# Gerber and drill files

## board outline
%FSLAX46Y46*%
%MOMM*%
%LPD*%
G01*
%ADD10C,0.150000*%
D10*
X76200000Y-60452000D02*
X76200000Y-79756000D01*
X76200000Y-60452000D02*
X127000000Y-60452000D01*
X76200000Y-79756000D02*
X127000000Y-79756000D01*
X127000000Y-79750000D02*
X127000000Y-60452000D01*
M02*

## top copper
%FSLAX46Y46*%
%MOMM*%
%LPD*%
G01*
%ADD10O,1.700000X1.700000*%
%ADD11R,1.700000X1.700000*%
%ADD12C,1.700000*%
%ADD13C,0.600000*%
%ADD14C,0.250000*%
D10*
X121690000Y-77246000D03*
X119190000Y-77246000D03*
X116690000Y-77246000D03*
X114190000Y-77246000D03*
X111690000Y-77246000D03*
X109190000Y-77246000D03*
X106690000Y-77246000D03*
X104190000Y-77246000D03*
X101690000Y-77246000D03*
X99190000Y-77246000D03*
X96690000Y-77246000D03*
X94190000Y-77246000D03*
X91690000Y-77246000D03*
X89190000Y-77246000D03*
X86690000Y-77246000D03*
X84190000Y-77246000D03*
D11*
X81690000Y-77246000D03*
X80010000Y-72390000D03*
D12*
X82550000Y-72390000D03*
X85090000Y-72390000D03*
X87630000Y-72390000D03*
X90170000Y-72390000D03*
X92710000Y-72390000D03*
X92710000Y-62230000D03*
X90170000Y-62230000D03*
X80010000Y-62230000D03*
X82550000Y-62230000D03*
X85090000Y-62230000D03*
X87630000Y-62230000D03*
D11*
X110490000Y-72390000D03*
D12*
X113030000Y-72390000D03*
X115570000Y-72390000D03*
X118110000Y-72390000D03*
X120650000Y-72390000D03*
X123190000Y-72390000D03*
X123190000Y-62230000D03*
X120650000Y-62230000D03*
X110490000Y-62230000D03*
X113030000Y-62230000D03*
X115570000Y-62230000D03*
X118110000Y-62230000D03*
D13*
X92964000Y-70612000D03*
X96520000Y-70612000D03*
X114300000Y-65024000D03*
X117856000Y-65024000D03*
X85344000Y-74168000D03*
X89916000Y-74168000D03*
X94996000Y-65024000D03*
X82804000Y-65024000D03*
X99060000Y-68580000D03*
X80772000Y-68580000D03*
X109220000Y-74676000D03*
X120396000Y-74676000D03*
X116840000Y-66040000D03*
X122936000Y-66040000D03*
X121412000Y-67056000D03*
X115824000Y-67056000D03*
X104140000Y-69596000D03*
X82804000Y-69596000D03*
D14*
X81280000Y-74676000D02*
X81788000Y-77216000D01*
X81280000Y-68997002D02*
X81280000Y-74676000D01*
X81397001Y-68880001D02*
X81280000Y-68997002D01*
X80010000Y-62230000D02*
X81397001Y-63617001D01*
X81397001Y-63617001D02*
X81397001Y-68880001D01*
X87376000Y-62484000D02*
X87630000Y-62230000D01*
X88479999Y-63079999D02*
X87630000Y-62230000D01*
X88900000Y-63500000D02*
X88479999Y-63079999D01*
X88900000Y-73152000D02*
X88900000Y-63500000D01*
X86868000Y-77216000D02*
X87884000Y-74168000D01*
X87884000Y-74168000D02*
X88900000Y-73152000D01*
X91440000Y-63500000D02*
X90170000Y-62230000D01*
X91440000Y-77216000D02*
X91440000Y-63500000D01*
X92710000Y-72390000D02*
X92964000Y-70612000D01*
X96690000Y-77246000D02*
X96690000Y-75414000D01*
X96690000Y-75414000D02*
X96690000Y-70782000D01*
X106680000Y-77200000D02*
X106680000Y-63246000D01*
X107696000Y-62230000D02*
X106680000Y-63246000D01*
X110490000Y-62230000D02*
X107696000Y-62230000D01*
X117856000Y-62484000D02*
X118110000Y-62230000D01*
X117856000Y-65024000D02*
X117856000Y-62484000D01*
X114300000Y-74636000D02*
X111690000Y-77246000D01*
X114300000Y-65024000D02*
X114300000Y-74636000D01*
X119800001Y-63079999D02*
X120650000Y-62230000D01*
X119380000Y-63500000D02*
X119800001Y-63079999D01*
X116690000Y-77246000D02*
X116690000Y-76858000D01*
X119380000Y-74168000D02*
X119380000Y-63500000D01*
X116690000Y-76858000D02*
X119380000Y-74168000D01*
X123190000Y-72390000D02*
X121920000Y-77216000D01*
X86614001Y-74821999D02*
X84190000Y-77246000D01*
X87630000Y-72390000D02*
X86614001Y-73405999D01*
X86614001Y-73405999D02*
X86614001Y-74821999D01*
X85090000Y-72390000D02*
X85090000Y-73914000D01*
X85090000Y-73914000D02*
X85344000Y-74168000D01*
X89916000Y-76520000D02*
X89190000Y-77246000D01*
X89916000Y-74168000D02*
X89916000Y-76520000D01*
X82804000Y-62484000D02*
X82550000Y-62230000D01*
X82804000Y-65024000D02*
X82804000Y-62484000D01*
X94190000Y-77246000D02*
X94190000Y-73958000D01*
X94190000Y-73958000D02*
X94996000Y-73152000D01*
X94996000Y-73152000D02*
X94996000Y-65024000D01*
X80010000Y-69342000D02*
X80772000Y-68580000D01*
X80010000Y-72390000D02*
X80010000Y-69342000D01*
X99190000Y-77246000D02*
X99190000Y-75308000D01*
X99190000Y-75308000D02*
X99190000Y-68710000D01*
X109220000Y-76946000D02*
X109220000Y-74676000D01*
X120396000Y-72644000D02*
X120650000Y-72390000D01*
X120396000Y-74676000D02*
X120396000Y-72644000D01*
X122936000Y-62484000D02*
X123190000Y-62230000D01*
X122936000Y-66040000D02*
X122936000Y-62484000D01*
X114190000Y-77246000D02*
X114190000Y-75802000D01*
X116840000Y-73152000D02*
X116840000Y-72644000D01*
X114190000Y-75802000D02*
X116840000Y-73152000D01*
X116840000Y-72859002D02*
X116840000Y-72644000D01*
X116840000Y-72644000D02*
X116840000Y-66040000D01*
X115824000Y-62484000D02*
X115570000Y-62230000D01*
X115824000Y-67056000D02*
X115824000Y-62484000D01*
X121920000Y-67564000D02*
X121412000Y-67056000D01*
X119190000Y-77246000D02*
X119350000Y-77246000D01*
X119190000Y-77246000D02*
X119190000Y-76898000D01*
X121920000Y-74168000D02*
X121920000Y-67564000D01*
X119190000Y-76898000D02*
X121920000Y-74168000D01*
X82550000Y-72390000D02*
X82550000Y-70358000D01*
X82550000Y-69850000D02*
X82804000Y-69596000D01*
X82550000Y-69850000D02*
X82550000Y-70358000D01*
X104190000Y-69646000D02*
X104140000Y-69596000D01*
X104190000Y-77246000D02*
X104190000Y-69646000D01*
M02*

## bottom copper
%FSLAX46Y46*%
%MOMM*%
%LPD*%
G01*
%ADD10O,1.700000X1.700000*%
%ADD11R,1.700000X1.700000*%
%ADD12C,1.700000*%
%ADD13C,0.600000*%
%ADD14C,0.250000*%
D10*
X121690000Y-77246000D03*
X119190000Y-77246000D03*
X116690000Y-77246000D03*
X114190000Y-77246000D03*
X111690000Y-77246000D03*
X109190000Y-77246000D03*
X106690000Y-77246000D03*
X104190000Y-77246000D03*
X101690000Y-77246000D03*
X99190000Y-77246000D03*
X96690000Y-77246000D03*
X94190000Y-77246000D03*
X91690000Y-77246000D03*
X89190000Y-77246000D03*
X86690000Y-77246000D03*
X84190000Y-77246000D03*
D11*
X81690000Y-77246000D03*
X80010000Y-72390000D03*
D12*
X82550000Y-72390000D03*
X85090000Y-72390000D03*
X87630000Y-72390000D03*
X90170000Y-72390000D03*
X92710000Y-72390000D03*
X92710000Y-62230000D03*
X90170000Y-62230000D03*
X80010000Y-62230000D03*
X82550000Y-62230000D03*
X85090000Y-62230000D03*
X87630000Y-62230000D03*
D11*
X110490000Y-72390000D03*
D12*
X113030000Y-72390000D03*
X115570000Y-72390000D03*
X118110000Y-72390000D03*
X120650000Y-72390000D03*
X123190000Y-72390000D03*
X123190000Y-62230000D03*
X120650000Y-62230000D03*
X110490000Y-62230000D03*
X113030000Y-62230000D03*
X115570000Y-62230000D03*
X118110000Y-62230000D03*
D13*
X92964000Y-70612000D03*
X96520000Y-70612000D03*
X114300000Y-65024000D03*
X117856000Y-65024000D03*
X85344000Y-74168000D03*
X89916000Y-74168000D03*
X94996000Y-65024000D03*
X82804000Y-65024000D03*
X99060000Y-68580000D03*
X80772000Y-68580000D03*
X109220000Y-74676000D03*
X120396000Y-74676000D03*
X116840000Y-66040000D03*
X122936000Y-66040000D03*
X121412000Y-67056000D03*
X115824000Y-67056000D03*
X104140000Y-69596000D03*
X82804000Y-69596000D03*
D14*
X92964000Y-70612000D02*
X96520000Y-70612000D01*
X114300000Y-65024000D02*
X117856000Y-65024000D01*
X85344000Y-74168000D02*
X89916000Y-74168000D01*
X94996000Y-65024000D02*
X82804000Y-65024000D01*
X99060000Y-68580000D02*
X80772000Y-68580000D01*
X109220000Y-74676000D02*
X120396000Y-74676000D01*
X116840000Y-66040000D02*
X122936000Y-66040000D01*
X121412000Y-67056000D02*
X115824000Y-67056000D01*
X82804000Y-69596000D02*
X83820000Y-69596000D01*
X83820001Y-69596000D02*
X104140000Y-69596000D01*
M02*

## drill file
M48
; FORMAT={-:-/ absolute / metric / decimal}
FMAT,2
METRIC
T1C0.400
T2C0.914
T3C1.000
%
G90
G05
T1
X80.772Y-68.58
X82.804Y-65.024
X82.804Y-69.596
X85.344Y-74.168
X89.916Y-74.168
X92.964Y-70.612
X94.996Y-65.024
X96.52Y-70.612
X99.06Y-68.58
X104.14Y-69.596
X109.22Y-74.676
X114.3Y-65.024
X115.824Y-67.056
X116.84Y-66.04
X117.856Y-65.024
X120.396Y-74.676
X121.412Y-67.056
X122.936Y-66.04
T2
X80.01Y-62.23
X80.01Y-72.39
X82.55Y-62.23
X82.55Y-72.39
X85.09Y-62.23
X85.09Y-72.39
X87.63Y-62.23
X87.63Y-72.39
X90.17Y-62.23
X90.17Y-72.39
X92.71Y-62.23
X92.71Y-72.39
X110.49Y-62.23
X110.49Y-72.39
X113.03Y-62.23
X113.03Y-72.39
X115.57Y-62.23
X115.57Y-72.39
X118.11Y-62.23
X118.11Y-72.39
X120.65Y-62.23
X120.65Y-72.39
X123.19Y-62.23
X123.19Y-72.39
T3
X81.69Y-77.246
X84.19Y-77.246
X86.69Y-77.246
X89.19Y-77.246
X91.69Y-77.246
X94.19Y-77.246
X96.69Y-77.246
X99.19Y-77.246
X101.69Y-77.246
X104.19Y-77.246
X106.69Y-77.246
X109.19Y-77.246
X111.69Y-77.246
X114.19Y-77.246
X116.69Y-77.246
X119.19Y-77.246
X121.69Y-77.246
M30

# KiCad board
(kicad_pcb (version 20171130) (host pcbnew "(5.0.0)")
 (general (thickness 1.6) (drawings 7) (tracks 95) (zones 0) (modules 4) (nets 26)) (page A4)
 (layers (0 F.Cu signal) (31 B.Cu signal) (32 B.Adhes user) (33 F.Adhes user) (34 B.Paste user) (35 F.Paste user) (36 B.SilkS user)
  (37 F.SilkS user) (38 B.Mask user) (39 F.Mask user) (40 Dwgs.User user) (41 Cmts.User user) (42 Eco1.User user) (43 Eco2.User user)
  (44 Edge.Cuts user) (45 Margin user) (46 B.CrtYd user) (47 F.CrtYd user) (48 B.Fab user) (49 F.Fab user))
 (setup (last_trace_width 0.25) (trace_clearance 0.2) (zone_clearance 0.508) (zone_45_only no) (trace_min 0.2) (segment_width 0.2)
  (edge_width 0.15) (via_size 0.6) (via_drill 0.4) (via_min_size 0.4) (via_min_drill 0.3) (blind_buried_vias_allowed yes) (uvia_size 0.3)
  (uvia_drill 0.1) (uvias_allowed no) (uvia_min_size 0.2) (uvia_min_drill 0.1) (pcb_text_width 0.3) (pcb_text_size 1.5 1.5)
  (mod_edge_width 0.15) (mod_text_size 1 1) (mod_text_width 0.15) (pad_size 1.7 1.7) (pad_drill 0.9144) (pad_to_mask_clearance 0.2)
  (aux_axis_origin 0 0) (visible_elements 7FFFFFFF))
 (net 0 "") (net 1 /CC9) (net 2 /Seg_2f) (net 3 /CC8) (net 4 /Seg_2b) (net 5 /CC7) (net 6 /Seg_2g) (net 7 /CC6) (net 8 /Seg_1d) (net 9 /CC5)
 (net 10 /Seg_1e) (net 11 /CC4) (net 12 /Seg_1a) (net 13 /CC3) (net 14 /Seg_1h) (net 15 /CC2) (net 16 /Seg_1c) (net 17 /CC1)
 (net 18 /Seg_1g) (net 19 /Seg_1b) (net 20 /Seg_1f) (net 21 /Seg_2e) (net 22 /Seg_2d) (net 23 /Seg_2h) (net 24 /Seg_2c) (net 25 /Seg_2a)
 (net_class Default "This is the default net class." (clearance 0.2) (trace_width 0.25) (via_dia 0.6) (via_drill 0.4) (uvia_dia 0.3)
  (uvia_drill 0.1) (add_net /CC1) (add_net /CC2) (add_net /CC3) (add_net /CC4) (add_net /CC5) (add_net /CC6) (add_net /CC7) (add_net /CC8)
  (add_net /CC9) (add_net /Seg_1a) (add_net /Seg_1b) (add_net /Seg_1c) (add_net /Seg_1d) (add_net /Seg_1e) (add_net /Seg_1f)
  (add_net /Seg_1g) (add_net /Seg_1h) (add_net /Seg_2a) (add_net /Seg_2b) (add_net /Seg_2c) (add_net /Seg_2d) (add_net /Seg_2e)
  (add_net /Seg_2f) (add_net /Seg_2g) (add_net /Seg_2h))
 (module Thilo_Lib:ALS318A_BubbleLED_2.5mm (layer F.Cu) (at 102.87 77.216)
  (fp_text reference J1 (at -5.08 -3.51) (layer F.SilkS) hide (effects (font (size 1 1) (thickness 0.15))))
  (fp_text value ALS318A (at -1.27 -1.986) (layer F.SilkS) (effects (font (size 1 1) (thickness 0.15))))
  (pad 17 thru_hole oval (at 18.82 0.03 90) (size 1.7 1.7) (drill 1) (layers *.Cu *.Mask) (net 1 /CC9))
  (pad 16 thru_hole oval (at 16.32 0.03 90) (size 1.7 1.7) (drill 1) (layers *.Cu *.Mask) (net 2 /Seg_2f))
  (pad 15 thru_hole oval (at 13.82 0.03 90) (size 1.7 1.7) (drill 1) (layers *.Cu *.Mask) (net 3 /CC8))
  (pad 14 thru_hole oval (at 11.32 0.03 90) (size 1.7 1.7) (drill 1) (layers *.Cu *.Mask) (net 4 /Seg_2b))
  (pad 13 thru_hole oval (at 8.82 0.03 90) (size 1.7 1.7) (drill 1) (layers *.Cu *.Mask) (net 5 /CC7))
  (pad 12 thru_hole oval (at 6.32 0.03 90) (size 1.7 1.7) (drill 1) (layers *.Cu *.Mask) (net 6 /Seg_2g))
  (pad 11 thru_hole oval (at 3.82 0.03 90) (size 1.7 1.7) (drill 1) (layers *.Cu *.Mask) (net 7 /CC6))
  (pad 10 thru_hole oval (at 1.32 0.03 90) (size 1.7 1.7) (drill 1) (layers *.Cu *.Mask) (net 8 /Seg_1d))
  (pad 9 thru_hole oval (at -1.18 0.03 90) (size 1.7 1.7) (drill 1) (layers *.Cu *.Mask) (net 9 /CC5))
  (pad 8 thru_hole oval (at -3.68 0.03 90) (size 1.7 1.7) (drill 1) (layers *.Cu *.Mask) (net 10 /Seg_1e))
  (pad 7 thru_hole oval (at -6.18 0.03 90) (size 1.7 1.7) (drill 1) (layers *.Cu *.Mask) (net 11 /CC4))
  (pad 6 thru_hole oval (at -8.68 0.03 90) (size 1.7 1.7) (drill 1) (layers *.Cu *.Mask) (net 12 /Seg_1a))
  (pad 5 thru_hole oval (at -11.18 0.03 90) (size 1.7 1.7) (drill 1) (layers *.Cu *.Mask) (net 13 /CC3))
  (pad 4 thru_hole oval (at -13.68 0.03 90) (size 1.7 1.7) (drill 1) (layers *.Cu *.Mask) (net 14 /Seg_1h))
  (pad 3 thru_hole oval (at -16.18 0.03 90) (size 1.7 1.7) (drill 1) (layers *.Cu *.Mask) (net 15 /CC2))
  (pad 2 thru_hole oval (at -18.68 0.03 90) (size 1.7 1.7) (drill 1) (layers *.Cu *.Mask) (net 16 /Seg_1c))
  (pad 1 thru_hole rect (at -21.18 0.03 90) (size 1.7 1.7) (drill 1) (layers *.Cu *.Mask) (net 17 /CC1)))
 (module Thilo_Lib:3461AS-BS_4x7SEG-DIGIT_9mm (layer F.Cu) (at 86.36 67.31)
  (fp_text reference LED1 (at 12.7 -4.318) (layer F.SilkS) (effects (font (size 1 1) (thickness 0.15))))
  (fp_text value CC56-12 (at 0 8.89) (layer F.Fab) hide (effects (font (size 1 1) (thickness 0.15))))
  (pad 1 thru_hole rect (at -6.35 5.08) (size 1.7 1.7) (drill 0.9144) (layers *.Cu *.Mask) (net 10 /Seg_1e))
  (pad 2 thru_hole circle (at -3.81 5.08) (size 1.7 1.7) (drill 0.9144) (layers *.Cu *.Mask) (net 8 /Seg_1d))
  (pad 3 thru_hole circle (at -1.27 5.08) (size 1.7 1.7) (drill 0.9144) (layers *.Cu *.Mask) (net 14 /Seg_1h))
  (pad 4 thru_hole circle (at 1.27 5.08) (size 1.7 1.7) (drill 0.9144) (layers *.Cu *.Mask) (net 16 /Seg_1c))
  (pad 5 thru_hole circle (at 3.81 5.08) (size 1.7 1.7) (drill 0.9144) (layers *.Cu *.Mask) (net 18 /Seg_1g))
  (pad 6 thru_hole circle (at 6.35 5.08) (size 1.7 1.7) (drill 0.9144) (layers *.Cu *.Mask) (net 11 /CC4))
  (pad 7 thru_hole circle (at 6.35 -5.08) (size 1.7 1.7) (drill 0.9144) (layers *.Cu *.Mask) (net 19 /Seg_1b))
  (pad 8 thru_hole circle (at 3.81 -5.08) (size 1.7 1.7) (drill 0.9144) (layers *.Cu *.Mask) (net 13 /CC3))
  (pad 12 thru_hole circle (at -6.35 -5.08) (size 1.7 1.7) (drill 0.9144) (layers *.Cu *.Mask) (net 17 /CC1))
  (pad 11 thru_hole circle (at -3.81 -5.08) (size 1.7 1.7) (drill 0.9144) (layers *.Cu *.Mask) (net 12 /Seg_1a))
  (pad 10 thru_hole circle (at -1.27 -5.08) (size 1.7 1.7) (drill 0.9144) (layers *.Cu *.Mask) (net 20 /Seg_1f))
  (pad 9 thru_hole circle (at 1.27 -5.08) (size 1.7 1.7) (drill 0.9144) (layers *.Cu *.Mask) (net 15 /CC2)))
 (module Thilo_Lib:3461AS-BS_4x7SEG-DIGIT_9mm (layer F.Cu) (at 116.84 67.31)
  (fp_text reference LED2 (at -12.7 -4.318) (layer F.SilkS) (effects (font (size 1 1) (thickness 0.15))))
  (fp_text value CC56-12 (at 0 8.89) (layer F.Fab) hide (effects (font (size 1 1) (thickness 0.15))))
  (pad 1 thru_hole rect (at -6.35 5.08) (size 1.7 1.7) (drill 0.9144) (layers *.Cu *.Mask) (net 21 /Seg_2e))
  (pad 2 thru_hole circle (at -3.81 5.08) (size 1.7 1.7) (drill 0.9144) (layers *.Cu *.Mask) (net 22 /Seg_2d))
  (pad 3 thru_hole circle (at -1.27 5.08) (size 1.7 1.7) (drill 0.9144) (layers *.Cu *.Mask) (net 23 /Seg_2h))
  (pad 4 thru_hole circle (at 1.27 5.08) (size 1.7 1.7) (drill 0.9144) (layers *.Cu *.Mask) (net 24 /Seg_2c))
  (pad 5 thru_hole circle (at 3.81 5.08) (size 1.7 1.7) (drill 0.9144) (layers *.Cu *.Mask) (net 6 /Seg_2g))
  (pad 6 thru_hole circle (at 6.35 5.08) (size 1.7 1.7) (drill 0.9144) (layers *.Cu *.Mask) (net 1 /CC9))
  (pad 7 thru_hole circle (at 6.35 -5.08) (size 1.7 1.7) (drill 0.9144) (layers *.Cu *.Mask) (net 4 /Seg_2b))
  (pad 8 thru_hole circle (at 3.81 -5.08) (size 1.7 1.7) (drill 0.9144) (layers *.Cu *.Mask) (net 3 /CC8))
  (pad 12 thru_hole circle (at -6.35 -5.08) (size 1.7 1.7) (drill 0.9144) (layers *.Cu *.Mask) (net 7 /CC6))
  (pad 11 thru_hole circle (at -3.81 -5.08) (size 1.7 1.7) (drill 0.9144) (layers *.Cu *.Mask) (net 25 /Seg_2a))
  (pad 10 thru_hole circle (at -1.27 -5.08) (size 1.7 1.7) (drill 0.9144) (layers *.Cu *.Mask) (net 2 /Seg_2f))
  (pad 9 thru_hole circle (at 1.27 -5.08) (size 1.7 1.7) (drill 0.9144) (layers *.Cu *.Mask) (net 5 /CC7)))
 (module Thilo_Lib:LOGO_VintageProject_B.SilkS (layer F.Cu) (at 115.824 69.596)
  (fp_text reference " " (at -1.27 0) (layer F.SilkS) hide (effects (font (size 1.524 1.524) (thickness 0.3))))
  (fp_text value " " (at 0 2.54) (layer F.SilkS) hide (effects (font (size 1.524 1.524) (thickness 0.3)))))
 (gr_line (start 76.2 60.452) (end 76.2 79.756) (layer Edge.Cuts) (width 0.15))
 (gr_line (start 76.2 60.452) (end 127 60.452) (layer Edge.Cuts) (width 0.15))
 (gr_line (start 76.2 79.756) (end 127 79.756) (layer Edge.Cuts) (width 0.15))
 (gr_line (start 127 79.75) (end 127 60.452) (angle 90) (layer Edge.Cuts) (width 0.15))
 (segment (start 81.28 74.676) (end 81.788 77.216) (width 0.25) (layer F.Cu) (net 17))
 (segment (start 81.28 68.997002) (end 81.28 74.676) (width 0.25) (layer F.Cu) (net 17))
 (segment (start 81.397001 68.880001) (end 81.28 68.997002) (width 0.25) (layer F.Cu) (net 17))
 (segment (start 80.01 62.23) (end 81.397001 63.617001) (width 0.25) (layer F.Cu) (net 17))
 (segment (start 81.397001 63.617001) (end 81.397001 68.880001) (width 0.25) (layer F.Cu) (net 17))
 (segment (start 87.376 62.484) (end 87.63 62.23) (width 0.25) (layer F.Cu) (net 15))
 (segment (start 88.479999 63.079999) (end 87.63 62.23) (width 0.25) (layer F.Cu) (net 15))
 (segment (start 88.9 63.5) (end 88.479999 63.079999) (width 0.25) (layer F.Cu) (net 15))
 (segment (start 88.9 73.152) (end 88.9 63.5) (width 0.25) (layer F.Cu) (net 15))
 (segment (start 86.868 77.216) (end 87.884 74.168) (width 0.25) (layer F.Cu) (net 15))
 (segment (start 87.884 74.168) (end 88.9 73.152) (width 0.25) (layer F.Cu) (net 15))
 (segment (start 91.44 63.5) (end 90.17 62.23) (width 0.25) (layer F.Cu) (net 13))
 (segment (start 91.44 77.216) (end 91.44 63.5) (width 0.25) (layer F.Cu) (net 13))
 (via blind (at 92.964 70.612) (size 0.6) (drill 0.4) (layers F.Cu B.Cu) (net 11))
 (via blind (at 96.52 70.612) (size 0.6) (drill 0.4) (layers F.Cu B.Cu) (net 11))
 (segment (start 92.71 72.39) (end 92.964 70.612) (width 0.25) (layer F.Cu) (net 11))
 (segment (start 96.69 77.246) (end 96.69 75.414) (width 0.25) (layer F.Cu) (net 11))
 (segment (start 96.69 75.414) (end 96.69 70.782) (width 0.25) (layer F.Cu) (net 11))
 (segment (start 92.964 70.612) (end 96.52 70.612) (width 0.25) (layer B.Cu) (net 11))
 (segment (start 106.68 77.2) (end 106.68 63.246) (width 0.25) (layer F.Cu) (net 7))
 (segment (start 107.696 62.23) (end 106.68 63.246) (width 0.25) (layer F.Cu) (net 7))
 (segment (start 110.49 62.23) (end 107.696 62.23) (width 0.25) (layer F.Cu) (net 7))
 (via blind (at 114.3 65.024) (size 0.6) (drill 0.4) (layers F.Cu B.Cu) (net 5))
 (segment (start 114.3 65.024) (end 117.856 65.024) (width 0.25) (layer B.Cu) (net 5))
 (via blind (at 117.856 65.024) (size 0.6) (drill 0.4) (layers F.Cu B.Cu) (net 5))
 (segment (start 117.856 62.484) (end 118.11 62.23) (width 0.25) (layer F.Cu) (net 5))
 (segment (start 117.856 65.024) (end 117.856 62.484) (width 0.25) (layer F.Cu) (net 5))
 (segment (start 114.3 74.636) (end 111.69 77.246) (width 0.25) (layer F.Cu) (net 5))
 (segment (start 114.3 65.024) (end 114.3 74.636) (width 0.25) (layer F.Cu) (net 5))
 (segment (start 119.800001 63.079999) (end 120.65 62.23) (width 0.25) (layer F.Cu) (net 3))
 (segment (start 119.38 63.5) (end 119.800001 63.079999) (width 0.25) (layer F.Cu) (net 3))
 (segment (start 116.69 77.246) (end 116.69 76.858) (width 0.25) (layer F.Cu) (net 3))
 (segment (start 119.38 74.168) (end 119.38 63.5) (width 0.25) (layer F.Cu) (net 3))
 (segment (start 116.69 76.858) (end 119.38 74.168) (width 0.25) (layer F.Cu) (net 3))
 (segment (start 123.19 72.39) (end 121.92 77.216) (width 0.25) (layer F.Cu) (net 1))
 (segment (start 86.614001 74.821999) (end 84.19 77.246) (width 0.25) (layer F.Cu) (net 16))
 (segment (start 87.63 72.39) (end 86.614001 73.405999) (width 0.25) (layer F.Cu) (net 16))
 (segment (start 86.614001 73.405999) (end 86.614001 74.821999) (width 0.25) (layer F.Cu) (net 16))
 (via blind (at 85.344 74.168) (size 0.6) (drill 0.4) (layers F.Cu B.Cu) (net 14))
 (segment (start 85.09 72.39) (end 85.09 73.914) (width 0.25) (layer F.Cu) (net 14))
 (segment (start 85.09 73.914) (end 85.344 74.168) (width 0.25) (layer F.Cu) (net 14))
 (via blind (at 89.916 74.168) (size 0.6) (drill 0.4) (layers F.Cu B.Cu) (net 14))
 (segment (start 85.344 74.168) (end 89.916 74.168) (width 0.25) (layer B.Cu) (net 14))
 (segment (start 89.916 76.52) (end 89.19 77.246) (width 0.25) (layer F.Cu) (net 14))
 (segment (start 89.916 74.168) (end 89.916 76.52) (width 0.25) (layer F.Cu) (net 14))
 (via blind (at 94.996 65.024) (size 0.6) (drill 0.4) (layers F.Cu B.Cu) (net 12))
 (via blind (at 82.804 65.024) (size 0.6) (drill 0.4) (layers F.Cu B.Cu) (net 12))
 (segment (start 82.804 62.484) (end 82.55 62.23) (width 0.25) (layer F.Cu) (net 12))
 (segment (start 82.804 65.024) (end 82.804 62.484) (width 0.25) (layer F.Cu) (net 12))
 (segment (start 94.19 77.246) (end 94.19 73.958) (width 0.25) (layer F.Cu) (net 12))
 (segment (start 94.19 73.958) (end 94.996 73.152) (width 0.25) (layer F.Cu) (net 12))
 (segment (start 94.996 73.152) (end 94.996 65.024) (width 0.25) (layer F.Cu) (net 12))
 (segment (start 94.996 65.024) (end 82.804 65.024) (width 0.25) (layer B.Cu) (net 12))
 (via blind (at 99.06 68.58) (size 0.6) (drill 0.4) (layers F.Cu B.Cu) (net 10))
 (via blind (at 80.772 68.58) (size 0.6) (drill 0.4) (layers F.Cu B.Cu) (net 10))
 (segment (start 80.01 69.342) (end 80.772 68.58) (width 0.25) (layer F.Cu) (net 10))
 (segment (start 80.01 72.39) (end 80.01 69.342) (width 0.25) (layer F.Cu) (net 10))
 (segment (start 99.19 77.246) (end 99.19 75.308) (width 0.25) (layer F.Cu) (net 10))
 (segment (start 99.19 75.308) (end 99.19 68.71) (width 0.25) (layer F.Cu) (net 10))
 (segment (start 99.06 68.58) (end 80.772 68.58) (width 0.25) (layer B.Cu) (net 10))
 (via blind (at 109.22 74.676) (size 0.6) (drill 0.4) (layers F.Cu B.Cu) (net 6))
 (segment (start 109.22 76.946) (end 109.22 74.676) (width 0.25) (layer F.Cu) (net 6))
 (via blind (at 120.396 74.676) (size 0.6) (drill 0.4) (layers F.Cu B.Cu) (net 6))
 (segment (start 120.396 72.644) (end 120.65 72.39) (width 0.25) (layer F.Cu) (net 6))
 (segment (start 120.396 74.676) (end 120.396 72.644) (width 0.25) (layer F.Cu) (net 6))
 (segment (start 109.22 74.676) (end 120.396 74.676) (width 0.25) (layer B.Cu) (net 6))
 (via blind (at 116.84 66.04) (size 0.6) (drill 0.4) (layers F.Cu B.Cu) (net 4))
 (via blind (at 122.936 66.04) (size 0.6) (drill 0.4) (layers F.Cu B.Cu) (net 4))
 (segment (start 116.84 66.04) (end 122.936 66.04) (width 0.25) (layer B.Cu) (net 4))
 (segment (start 122.936 62.484) (end 123.19 62.23) (width 0.25) (layer F.Cu) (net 4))
 (segment (start 122.936 66.04) (end 122.936 62.484) (width 0.25) (layer F.Cu) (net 4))
 (segment (start 114.19 77.246) (end 114.19 75.802) (width 0.25) (layer F.Cu) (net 4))
 (segment (start 116.84 73.152) (end 116.84 72.644) (width 0.25) (layer F.Cu) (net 4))
 (segment (start 114.19 75.802) (end 116.84 73.152) (width 0.25) (layer F.Cu) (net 4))
 (segment (start 116.84 72.859002) (end 116.84 72.644) (width 0.25) (layer F.Cu) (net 4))
 (segment (start 116.84 72.644) (end 116.84 66.04) (width 0.25) (layer F.Cu) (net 4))
 (via blind (at 121.412 67.056) (size 0.6) (drill 0.4) (layers F.Cu B.Cu) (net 2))
 (via blind (at 115.824 67.056) (size 0.6) (drill 0.4) (layers F.Cu B.Cu) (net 2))
 (segment (start 121.412 67.056) (end 115.824 67.056) (width 0.25) (layer B.Cu) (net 2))
 (segment (start 115.824 62.484) (end 115.57 62.23) (width 0.25) (layer F.Cu) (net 2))
 (segment (start 115.824 67.056) (end 115.824 62.484) (width 0.25) (layer F.Cu) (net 2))
 (segment (start 121.92 67.564) (end 121.412 67.056) (width 0.25) (layer F.Cu) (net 2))
 (segment (start 119.19 77.246) (end 119.35 77.246) (width 0.25) (layer F.Cu) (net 2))
 (segment (start 119.19 77.246) (end 119.19 76.898) (width 0.25) (layer F.Cu) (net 2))
 (segment (start 121.92 74.168) (end 121.92 67.564) (width 0.25) (layer F.Cu) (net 2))
 (segment (start 119.19 76.898) (end 121.92 74.168) (width 0.25) (layer F.Cu) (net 2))
 (via blind (at 104.14 69.596) (size 0.6) (drill 0.4) (layers F.Cu B.Cu) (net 8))
 (via blind (at 82.804 69.596) (size 0.6) (drill 0.4) (layers F.Cu B.Cu) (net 8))
 (segment (start 82.55 72.39) (end 82.55 70.358) (width 0.25) (layer F.Cu) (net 8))
 (segment (start 82.55 69.85) (end 82.804 69.596) (width 0.25) (layer F.Cu) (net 8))
 (segment (start 82.804 69.596) (end 83.82 69.596) (width 0.25) (layer B.Cu) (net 8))
 (segment (start 82.55 69.85) (end 82.55 70.358) (width 0.25) (layer F.Cu) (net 8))
 (segment (start 83.820001 69.596) (end 104.14 69.596) (width 0.25) (layer B.Cu) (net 8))
 (segment (start 104.19 69.646) (end 104.14 69.596) (width 0.25) (layer F.Cu) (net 8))
 (segment (start 104.19 77.246) (end 104.19 69.646) (width 0.25) (layer F.Cu) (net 8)))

